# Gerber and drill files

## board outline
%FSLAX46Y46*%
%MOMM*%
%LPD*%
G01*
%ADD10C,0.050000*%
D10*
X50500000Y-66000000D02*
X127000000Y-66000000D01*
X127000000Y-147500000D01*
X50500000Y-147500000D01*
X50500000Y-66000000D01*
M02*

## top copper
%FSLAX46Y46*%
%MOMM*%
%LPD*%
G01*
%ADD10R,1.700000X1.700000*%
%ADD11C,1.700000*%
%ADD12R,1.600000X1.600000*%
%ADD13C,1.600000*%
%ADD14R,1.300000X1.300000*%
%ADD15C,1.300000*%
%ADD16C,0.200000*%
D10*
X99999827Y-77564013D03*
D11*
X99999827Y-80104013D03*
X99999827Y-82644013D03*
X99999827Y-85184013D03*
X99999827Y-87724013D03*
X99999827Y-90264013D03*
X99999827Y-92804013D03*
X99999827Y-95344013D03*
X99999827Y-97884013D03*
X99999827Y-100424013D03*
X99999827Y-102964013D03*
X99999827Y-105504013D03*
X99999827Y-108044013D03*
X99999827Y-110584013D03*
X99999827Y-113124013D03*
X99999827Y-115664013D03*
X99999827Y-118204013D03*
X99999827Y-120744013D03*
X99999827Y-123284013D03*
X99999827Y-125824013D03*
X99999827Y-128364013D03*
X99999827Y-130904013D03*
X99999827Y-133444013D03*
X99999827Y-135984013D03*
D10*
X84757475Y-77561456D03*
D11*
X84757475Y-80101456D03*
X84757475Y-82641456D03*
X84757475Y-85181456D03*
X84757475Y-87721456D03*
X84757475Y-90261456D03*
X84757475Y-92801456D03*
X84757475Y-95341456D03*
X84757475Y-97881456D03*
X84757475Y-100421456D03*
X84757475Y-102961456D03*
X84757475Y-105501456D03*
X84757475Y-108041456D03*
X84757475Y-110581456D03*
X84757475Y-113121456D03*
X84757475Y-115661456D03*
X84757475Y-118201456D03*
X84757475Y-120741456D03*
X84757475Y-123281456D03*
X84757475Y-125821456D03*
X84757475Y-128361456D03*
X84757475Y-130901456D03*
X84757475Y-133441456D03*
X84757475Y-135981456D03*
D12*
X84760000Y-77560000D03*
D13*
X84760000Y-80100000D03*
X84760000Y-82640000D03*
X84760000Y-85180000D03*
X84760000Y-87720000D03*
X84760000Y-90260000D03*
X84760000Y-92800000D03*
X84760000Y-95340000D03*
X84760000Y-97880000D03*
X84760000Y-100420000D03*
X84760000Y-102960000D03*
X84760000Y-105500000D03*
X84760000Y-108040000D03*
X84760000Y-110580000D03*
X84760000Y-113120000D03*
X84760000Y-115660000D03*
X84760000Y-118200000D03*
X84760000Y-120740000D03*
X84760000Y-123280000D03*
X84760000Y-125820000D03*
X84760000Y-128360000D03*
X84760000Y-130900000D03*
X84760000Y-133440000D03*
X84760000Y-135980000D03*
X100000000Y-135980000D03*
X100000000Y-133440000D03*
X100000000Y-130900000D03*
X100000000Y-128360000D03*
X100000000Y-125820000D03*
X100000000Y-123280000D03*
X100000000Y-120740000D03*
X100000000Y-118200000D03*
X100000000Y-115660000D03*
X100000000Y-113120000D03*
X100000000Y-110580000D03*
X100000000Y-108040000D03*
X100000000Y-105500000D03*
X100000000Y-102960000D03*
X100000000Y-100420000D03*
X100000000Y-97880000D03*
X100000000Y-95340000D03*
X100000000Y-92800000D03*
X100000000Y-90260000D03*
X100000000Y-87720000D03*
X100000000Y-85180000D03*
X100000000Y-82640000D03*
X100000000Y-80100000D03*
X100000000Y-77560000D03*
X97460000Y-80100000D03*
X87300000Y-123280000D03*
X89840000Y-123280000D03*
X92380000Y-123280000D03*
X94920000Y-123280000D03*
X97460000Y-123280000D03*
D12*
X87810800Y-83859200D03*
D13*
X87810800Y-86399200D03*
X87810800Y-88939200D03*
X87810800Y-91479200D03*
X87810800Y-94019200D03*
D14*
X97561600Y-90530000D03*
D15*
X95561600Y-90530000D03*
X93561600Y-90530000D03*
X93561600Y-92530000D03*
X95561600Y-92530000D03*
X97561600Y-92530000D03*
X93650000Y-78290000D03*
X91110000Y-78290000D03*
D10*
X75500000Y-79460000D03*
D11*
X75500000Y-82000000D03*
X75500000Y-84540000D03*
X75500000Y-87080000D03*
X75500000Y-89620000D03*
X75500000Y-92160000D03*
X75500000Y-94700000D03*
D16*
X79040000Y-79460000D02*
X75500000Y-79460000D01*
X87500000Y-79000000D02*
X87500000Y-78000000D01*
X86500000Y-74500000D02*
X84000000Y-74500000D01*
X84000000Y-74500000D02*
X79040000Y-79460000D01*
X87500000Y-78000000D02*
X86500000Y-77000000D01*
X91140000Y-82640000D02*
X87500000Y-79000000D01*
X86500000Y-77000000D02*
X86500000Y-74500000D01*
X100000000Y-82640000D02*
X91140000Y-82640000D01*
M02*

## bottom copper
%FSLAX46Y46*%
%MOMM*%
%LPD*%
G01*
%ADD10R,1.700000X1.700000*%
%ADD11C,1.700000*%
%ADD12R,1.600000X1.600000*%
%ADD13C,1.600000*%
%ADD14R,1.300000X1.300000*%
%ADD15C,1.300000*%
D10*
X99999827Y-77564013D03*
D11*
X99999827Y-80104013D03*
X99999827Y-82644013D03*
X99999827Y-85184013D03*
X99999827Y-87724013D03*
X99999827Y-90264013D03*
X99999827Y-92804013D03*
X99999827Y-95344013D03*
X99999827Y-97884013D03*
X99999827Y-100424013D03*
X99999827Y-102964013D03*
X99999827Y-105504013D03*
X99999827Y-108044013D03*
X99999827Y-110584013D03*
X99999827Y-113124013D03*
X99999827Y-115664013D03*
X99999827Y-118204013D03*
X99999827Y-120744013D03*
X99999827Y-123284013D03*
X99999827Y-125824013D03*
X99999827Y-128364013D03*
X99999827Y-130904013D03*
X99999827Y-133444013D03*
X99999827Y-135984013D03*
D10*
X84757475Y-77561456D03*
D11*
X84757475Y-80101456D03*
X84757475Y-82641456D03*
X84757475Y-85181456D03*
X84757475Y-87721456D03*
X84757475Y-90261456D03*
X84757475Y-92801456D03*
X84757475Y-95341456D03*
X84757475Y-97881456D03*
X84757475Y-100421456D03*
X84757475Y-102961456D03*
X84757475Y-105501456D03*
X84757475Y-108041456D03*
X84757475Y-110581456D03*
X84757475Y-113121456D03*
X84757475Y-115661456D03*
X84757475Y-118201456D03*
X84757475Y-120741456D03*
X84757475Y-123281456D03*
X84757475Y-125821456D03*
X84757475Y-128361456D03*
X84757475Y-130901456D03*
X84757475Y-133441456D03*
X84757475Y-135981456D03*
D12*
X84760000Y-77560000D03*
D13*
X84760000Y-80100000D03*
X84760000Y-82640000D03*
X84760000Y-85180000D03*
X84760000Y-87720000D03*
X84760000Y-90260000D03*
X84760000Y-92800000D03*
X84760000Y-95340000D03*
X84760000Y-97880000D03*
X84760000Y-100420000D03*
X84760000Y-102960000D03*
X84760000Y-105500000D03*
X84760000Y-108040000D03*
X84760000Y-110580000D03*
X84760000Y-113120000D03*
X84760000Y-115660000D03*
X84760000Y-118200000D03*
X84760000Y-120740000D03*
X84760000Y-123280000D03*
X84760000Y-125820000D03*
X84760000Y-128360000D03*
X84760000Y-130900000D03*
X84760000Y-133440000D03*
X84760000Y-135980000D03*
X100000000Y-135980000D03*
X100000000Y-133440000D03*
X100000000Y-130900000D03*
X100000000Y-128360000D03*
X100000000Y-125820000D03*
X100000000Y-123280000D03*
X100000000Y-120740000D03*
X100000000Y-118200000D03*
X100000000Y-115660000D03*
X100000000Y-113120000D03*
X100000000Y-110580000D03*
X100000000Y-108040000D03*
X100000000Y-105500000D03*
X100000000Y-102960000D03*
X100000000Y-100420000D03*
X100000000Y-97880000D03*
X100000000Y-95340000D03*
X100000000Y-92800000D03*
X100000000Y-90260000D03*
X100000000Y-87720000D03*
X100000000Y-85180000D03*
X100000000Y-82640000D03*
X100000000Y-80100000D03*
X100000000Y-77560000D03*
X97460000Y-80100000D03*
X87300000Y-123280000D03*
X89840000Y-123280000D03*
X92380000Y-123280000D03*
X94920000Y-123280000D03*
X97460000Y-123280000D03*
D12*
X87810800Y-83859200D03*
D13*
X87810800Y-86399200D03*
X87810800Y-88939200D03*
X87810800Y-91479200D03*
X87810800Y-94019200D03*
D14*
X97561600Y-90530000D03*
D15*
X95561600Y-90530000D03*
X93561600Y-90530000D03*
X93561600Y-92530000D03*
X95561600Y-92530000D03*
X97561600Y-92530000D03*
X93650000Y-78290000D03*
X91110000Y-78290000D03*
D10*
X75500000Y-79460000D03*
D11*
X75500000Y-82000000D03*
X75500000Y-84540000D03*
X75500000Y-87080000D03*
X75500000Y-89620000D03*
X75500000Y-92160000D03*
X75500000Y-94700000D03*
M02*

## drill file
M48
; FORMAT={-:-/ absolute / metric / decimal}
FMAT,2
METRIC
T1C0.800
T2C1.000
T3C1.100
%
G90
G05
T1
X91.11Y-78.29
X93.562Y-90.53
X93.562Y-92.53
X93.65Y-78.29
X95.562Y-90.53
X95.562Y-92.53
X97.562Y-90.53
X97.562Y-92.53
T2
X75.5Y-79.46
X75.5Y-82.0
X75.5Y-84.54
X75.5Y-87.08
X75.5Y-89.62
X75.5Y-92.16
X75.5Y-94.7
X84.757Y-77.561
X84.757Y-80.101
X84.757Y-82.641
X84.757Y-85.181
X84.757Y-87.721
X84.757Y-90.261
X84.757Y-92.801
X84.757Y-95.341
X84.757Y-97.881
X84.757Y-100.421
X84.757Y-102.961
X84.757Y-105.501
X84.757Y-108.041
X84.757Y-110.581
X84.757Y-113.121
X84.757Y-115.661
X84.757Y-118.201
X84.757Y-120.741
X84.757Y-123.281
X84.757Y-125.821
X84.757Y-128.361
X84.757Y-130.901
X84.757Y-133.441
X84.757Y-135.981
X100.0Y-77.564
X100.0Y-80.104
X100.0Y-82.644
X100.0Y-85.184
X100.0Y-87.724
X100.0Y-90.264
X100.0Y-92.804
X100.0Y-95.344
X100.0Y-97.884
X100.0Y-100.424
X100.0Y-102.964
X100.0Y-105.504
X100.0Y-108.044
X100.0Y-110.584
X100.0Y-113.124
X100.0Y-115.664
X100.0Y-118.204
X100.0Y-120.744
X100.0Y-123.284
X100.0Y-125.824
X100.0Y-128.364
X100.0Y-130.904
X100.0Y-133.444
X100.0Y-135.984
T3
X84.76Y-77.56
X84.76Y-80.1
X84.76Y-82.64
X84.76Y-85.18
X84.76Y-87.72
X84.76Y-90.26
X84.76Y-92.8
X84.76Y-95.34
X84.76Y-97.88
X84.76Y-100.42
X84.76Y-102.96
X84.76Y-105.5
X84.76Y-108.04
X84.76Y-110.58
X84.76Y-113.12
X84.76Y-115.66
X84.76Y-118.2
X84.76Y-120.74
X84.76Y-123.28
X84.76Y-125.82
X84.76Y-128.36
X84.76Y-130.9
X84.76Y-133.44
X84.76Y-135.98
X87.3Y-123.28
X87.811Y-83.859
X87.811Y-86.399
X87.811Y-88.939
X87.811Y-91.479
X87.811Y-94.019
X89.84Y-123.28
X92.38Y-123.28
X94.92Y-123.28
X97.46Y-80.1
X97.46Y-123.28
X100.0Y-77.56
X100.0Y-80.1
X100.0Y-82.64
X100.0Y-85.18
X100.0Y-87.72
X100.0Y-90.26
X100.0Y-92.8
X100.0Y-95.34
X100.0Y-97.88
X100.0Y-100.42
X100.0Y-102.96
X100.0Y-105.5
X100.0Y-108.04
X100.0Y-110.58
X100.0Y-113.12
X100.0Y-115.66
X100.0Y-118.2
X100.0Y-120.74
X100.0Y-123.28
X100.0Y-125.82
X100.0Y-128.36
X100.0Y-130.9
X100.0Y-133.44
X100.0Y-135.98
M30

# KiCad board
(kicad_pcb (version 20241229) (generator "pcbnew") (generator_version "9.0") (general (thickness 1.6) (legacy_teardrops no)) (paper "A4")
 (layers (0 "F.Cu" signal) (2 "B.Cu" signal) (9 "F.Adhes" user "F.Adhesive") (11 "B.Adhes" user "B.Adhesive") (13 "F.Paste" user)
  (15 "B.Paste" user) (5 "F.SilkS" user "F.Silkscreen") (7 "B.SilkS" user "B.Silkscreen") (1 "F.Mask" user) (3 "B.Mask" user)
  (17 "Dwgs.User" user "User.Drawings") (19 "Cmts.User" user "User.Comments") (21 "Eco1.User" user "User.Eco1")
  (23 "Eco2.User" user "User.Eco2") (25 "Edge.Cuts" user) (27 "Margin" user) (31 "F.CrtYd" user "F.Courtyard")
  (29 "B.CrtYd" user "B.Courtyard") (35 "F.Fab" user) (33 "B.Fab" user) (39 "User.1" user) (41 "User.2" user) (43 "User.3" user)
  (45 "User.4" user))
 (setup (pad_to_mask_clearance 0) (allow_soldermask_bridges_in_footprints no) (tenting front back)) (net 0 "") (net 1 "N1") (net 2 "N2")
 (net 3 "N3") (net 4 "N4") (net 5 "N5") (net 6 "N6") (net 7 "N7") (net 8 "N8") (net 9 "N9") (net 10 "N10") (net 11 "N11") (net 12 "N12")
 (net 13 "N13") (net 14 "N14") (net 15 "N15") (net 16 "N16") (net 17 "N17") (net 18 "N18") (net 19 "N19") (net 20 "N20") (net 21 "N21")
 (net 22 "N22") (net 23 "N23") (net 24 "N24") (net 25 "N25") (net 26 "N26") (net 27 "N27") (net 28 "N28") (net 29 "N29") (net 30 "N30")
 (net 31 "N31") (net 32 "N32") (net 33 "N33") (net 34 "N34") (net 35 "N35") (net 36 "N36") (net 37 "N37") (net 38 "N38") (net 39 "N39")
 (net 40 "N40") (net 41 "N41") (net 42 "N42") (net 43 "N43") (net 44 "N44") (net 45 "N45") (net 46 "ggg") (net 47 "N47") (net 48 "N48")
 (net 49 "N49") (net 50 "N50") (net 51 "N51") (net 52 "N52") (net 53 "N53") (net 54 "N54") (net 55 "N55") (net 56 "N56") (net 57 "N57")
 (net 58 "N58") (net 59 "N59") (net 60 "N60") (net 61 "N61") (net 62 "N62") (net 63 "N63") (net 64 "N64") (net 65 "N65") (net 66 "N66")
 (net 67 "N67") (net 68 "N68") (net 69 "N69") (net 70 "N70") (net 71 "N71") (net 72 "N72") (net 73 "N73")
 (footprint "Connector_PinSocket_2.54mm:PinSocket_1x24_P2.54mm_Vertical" (layer "F.Cu") (at 99.999827 77.564013)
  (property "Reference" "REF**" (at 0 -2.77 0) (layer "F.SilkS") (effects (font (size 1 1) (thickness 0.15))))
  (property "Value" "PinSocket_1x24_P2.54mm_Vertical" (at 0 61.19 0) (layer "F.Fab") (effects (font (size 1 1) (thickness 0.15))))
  (pad "1" thru_hole rect (at 0 0) (size 1.7 1.7) (drill 1) (layers "*.Cu" "*.Mask") (remove_unused_layers no))
  (pad "2" thru_hole circle (at 0 2.54) (size 1.7 1.7) (drill 1) (layers "*.Cu" "*.Mask") (remove_unused_layers no))
  (pad "3" thru_hole circle (at 0 5.08) (size 1.7 1.7) (drill 1) (layers "*.Cu" "*.Mask") (remove_unused_layers no))
  (pad "4" thru_hole circle (at 0 7.62) (size 1.7 1.7) (drill 1) (layers "*.Cu" "*.Mask") (remove_unused_layers no))
  (pad "5" thru_hole circle (at 0 10.16) (size 1.7 1.7) (drill 1) (layers "*.Cu" "*.Mask") (remove_unused_layers no))
  (pad "6" thru_hole circle (at 0 12.7) (size 1.7 1.7) (drill 1) (layers "*.Cu" "*.Mask") (remove_unused_layers no))
  (pad "7" thru_hole circle (at 0 15.24) (size 1.7 1.7) (drill 1) (layers "*.Cu" "*.Mask") (remove_unused_layers no))
  (pad "8" thru_hole circle (at 0 17.78) (size 1.7 1.7) (drill 1) (layers "*.Cu" "*.Mask") (remove_unused_layers no))
  (pad "9" thru_hole circle (at 0 20.32) (size 1.7 1.7) (drill 1) (layers "*.Cu" "*.Mask") (remove_unused_layers no))
  (pad "10" thru_hole circle (at 0 22.86) (size 1.7 1.7) (drill 1) (layers "*.Cu" "*.Mask") (remove_unused_layers no))
  (pad "11" thru_hole circle (at 0 25.4) (size 1.7 1.7) (drill 1) (layers "*.Cu" "*.Mask") (remove_unused_layers no))
  (pad "12" thru_hole circle (at 0 27.94) (size 1.7 1.7) (drill 1) (layers "*.Cu" "*.Mask") (remove_unused_layers no))
  (pad "13" thru_hole circle (at 0 30.48) (size 1.7 1.7) (drill 1) (layers "*.Cu" "*.Mask") (remove_unused_layers no))
  (pad "14" thru_hole circle (at 0 33.02) (size 1.7 1.7) (drill 1) (layers "*.Cu" "*.Mask") (remove_unused_layers no))
  (pad "15" thru_hole circle (at 0 35.56) (size 1.7 1.7) (drill 1) (layers "*.Cu" "*.Mask") (remove_unused_layers no))
  (pad "16" thru_hole circle (at 0 38.1) (size 1.7 1.7) (drill 1) (layers "*.Cu" "*.Mask") (remove_unused_layers no))
  (pad "17" thru_hole circle (at 0 40.64) (size 1.7 1.7) (drill 1) (layers "*.Cu" "*.Mask") (remove_unused_layers no))
  (pad "18" thru_hole circle (at 0 43.18) (size 1.7 1.7) (drill 1) (layers "*.Cu" "*.Mask") (remove_unused_layers no))
  (pad "19" thru_hole circle (at 0 45.72) (size 1.7 1.7) (drill 1) (layers "*.Cu" "*.Mask") (remove_unused_layers no))
  (pad "20" thru_hole circle (at 0 48.26) (size 1.7 1.7) (drill 1) (layers "*.Cu" "*.Mask") (remove_unused_layers no))
  (pad "21" thru_hole circle (at 0 50.8) (size 1.7 1.7) (drill 1) (layers "*.Cu" "*.Mask") (remove_unused_layers no))
  (pad "22" thru_hole circle (at 0 53.34) (size 1.7 1.7) (drill 1) (layers "*.Cu" "*.Mask") (remove_unused_layers no))
  (pad "23" thru_hole circle (at 0 55.88) (size 1.7 1.7) (drill 1) (layers "*.Cu" "*.Mask") (remove_unused_layers no))
  (pad "24" thru_hole circle (at 0 58.42) (size 1.7 1.7) (drill 1) (layers "*.Cu" "*.Mask") (remove_unused_layers no)))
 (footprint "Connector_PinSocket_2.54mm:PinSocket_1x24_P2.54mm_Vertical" (layer "F.Cu") (at 84.757475 77.561456)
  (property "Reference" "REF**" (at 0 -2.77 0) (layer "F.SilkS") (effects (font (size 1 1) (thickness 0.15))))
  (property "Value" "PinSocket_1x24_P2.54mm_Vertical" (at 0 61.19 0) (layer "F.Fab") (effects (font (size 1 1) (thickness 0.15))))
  (pad "1" thru_hole rect (at 0 0) (size 1.7 1.7) (drill 1) (layers "*.Cu" "*.Mask") (remove_unused_layers no))
  (pad "2" thru_hole circle (at 0 2.54) (size 1.7 1.7) (drill 1) (layers "*.Cu" "*.Mask") (remove_unused_layers no))
  (pad "3" thru_hole circle (at 0 5.08) (size 1.7 1.7) (drill 1) (layers "*.Cu" "*.Mask") (remove_unused_layers no))
  (pad "4" thru_hole circle (at 0 7.62) (size 1.7 1.7) (drill 1) (layers "*.Cu" "*.Mask") (remove_unused_layers no))
  (pad "5" thru_hole circle (at 0 10.16) (size 1.7 1.7) (drill 1) (layers "*.Cu" "*.Mask") (remove_unused_layers no))
  (pad "6" thru_hole circle (at 0 12.7) (size 1.7 1.7) (drill 1) (layers "*.Cu" "*.Mask") (remove_unused_layers no))
  (pad "7" thru_hole circle (at 0 15.24) (size 1.7 1.7) (drill 1) (layers "*.Cu" "*.Mask") (remove_unused_layers no))
  (pad "8" thru_hole circle (at 0 17.78) (size 1.7 1.7) (drill 1) (layers "*.Cu" "*.Mask") (remove_unused_layers no))
  (pad "9" thru_hole circle (at 0 20.32) (size 1.7 1.7) (drill 1) (layers "*.Cu" "*.Mask") (remove_unused_layers no))
  (pad "10" thru_hole circle (at 0 22.86) (size 1.7 1.7) (drill 1) (layers "*.Cu" "*.Mask") (remove_unused_layers no))
  (pad "11" thru_hole circle (at 0 25.4) (size 1.7 1.7) (drill 1) (layers "*.Cu" "*.Mask") (remove_unused_layers no))
  (pad "12" thru_hole circle (at 0 27.94) (size 1.7 1.7) (drill 1) (layers "*.Cu" "*.Mask") (remove_unused_layers no))
  (pad "13" thru_hole circle (at 0 30.48) (size 1.7 1.7) (drill 1) (layers "*.Cu" "*.Mask") (remove_unused_layers no))
  (pad "14" thru_hole circle (at 0 33.02) (size 1.7 1.7) (drill 1) (layers "*.Cu" "*.Mask") (remove_unused_layers no))
  (pad "15" thru_hole circle (at 0 35.56) (size 1.7 1.7) (drill 1) (layers "*.Cu" "*.Mask") (remove_unused_layers no))
  (pad "16" thru_hole circle (at 0 38.1) (size 1.7 1.7) (drill 1) (layers "*.Cu" "*.Mask") (remove_unused_layers no))
  (pad "17" thru_hole circle (at 0 40.64) (size 1.7 1.7) (drill 1) (layers "*.Cu" "*.Mask") (remove_unused_layers no))
  (pad "18" thru_hole circle (at 0 43.18) (size 1.7 1.7) (drill 1) (layers "*.Cu" "*.Mask") (remove_unused_layers no))
  (pad "19" thru_hole circle (at 0 45.72) (size 1.7 1.7) (drill 1) (layers "*.Cu" "*.Mask") (remove_unused_layers no))
  (pad "20" thru_hole circle (at 0 48.26) (size 1.7 1.7) (drill 1) (layers "*.Cu" "*.Mask") (remove_unused_layers no))
  (pad "21" thru_hole circle (at 0 50.8) (size 1.7 1.7) (drill 1) (layers "*.Cu" "*.Mask") (remove_unused_layers no))
  (pad "22" thru_hole circle (at 0 53.34) (size 1.7 1.7) (drill 1) (layers "*.Cu" "*.Mask") (remove_unused_layers no))
  (pad "23" thru_hole circle (at 0 55.88) (size 1.7 1.7) (drill 1) (layers "*.Cu" "*.Mask") (remove_unused_layers no))
  (pad "24" thru_hole circle (at 0 58.42) (size 1.7 1.7) (drill 1) (layers "*.Cu" "*.Mask") (remove_unused_layers no)))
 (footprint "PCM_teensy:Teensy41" (layer "F.Cu") (at 92.38 106.77 -90)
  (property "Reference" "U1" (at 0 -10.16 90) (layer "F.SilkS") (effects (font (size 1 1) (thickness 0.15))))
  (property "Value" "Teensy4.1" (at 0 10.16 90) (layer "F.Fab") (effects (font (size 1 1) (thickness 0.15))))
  (pad "1" thru_hole rect (at -29.21 7.62 270) (size 1.6 1.6) (drill 1.1) (layers "*.Cu" "*.Mask") (remove_unused_layers no) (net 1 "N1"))
  (pad "2" thru_hole circle (at -26.67 7.62 270) (size 1.6 1.6) (drill 1.1) (layers "*.Cu" "*.Mask") (remove_unused_layers no) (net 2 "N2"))
  (pad "3" thru_hole circle (at -24.13 7.62 270) (size 1.6 1.6) (drill 1.1) (layers "*.Cu" "*.Mask") (remove_unused_layers no) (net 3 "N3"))
  (pad "4" thru_hole circle (at -21.59 7.62 270) (size 1.6 1.6) (drill 1.1) (layers "*.Cu" "*.Mask") (remove_unused_layers no) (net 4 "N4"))
  (pad "5" thru_hole circle (at -19.05 7.62 270) (size 1.6 1.6) (drill 1.1) (layers "*.Cu" "*.Mask") (remove_unused_layers no) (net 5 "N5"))
  (pad "6" thru_hole circle (at -16.51 7.62 270) (size 1.6 1.6) (drill 1.1) (layers "*.Cu" "*.Mask") (remove_unused_layers no) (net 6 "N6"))
  (pad "7" thru_hole circle (at -13.97 7.62 270) (size 1.6 1.6) (drill 1.1) (layers "*.Cu" "*.Mask") (remove_unused_layers no) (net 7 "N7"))
  (pad "8" thru_hole circle (at -11.43 7.62 270) (size 1.6 1.6) (drill 1.1) (layers "*.Cu" "*.Mask") (remove_unused_layers no) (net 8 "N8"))
  (pad "9" thru_hole circle (at -8.89 7.62 270) (size 1.6 1.6) (drill 1.1) (layers "*.Cu" "*.Mask") (remove_unused_layers no) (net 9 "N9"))
  (pad "10" thru_hole circle (at -6.35 7.62 270) (size 1.6 1.6) (drill 1.1) (layers "*.Cu" "*.Mask") (remove_unused_layers no)
   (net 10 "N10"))
  (pad "11" thru_hole circle (at -3.81 7.62 270) (size 1.6 1.6) (drill 1.1) (layers "*.Cu" "*.Mask") (remove_unused_layers no)
   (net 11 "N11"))
  (pad "12" thru_hole circle (at -1.27 7.62 270) (size 1.6 1.6) (drill 1.1) (layers "*.Cu" "*.Mask") (remove_unused_layers no)
   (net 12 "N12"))
  (pad "13" thru_hole circle (at 1.27 7.62 270) (size 1.6 1.6) (drill 1.1) (layers "*.Cu" "*.Mask") (remove_unused_layers no) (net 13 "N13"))
  (pad "14" thru_hole circle (at 3.81 7.62 270) (size 1.6 1.6) (drill 1.1) (layers "*.Cu" "*.Mask") (remove_unused_layers no) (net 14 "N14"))
  (pad "15" thru_hole circle (at 6.35 7.62 270) (size 1.6 1.6) (drill 1.1) (layers "*.Cu" "*.Mask") (remove_unused_layers no) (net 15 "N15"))
  (pad "16" thru_hole circle (at 8.89 7.62 270) (size 1.6 1.6) (drill 1.1) (layers "*.Cu" "*.Mask") (remove_unused_layers no) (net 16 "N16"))
  (pad "17" thru_hole circle (at 11.43 7.62 270) (size 1.6 1.6) (drill 1.1) (layers "*.Cu" "*.Mask") (remove_unused_layers no)
   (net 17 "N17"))
  (pad "18" thru_hole circle (at 13.97 7.62 270) (size 1.6 1.6) (drill 1.1) (layers "*.Cu" "*.Mask") (remove_unused_layers no)
   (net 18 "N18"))
  (pad "19" thru_hole circle (at 16.51 7.62 270) (size 1.6 1.6) (drill 1.1) (layers "*.Cu" "*.Mask") (remove_unused_layers no)
   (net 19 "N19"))
  (pad "20" thru_hole circle (at 19.05 7.62 270) (size 1.6 1.6) (drill 1.1) (layers "*.Cu" "*.Mask") (remove_unused_layers no)
   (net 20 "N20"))
  (pad "21" thru_hole circle (at 21.59 7.62 270) (size 1.6 1.6) (drill 1.1) (layers "*.Cu" "*.Mask") (remove_unused_layers no)
   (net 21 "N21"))
  (pad "22" thru_hole circle (at 24.13 7.62 270) (size 1.6 1.6) (drill 1.1) (layers "*.Cu" "*.Mask") (remove_unused_layers no)
   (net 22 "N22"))
  (pad "23" thru_hole circle (at 26.67 7.62 270) (size 1.6 1.6) (drill 1.1) (layers "*.Cu" "*.Mask") (remove_unused_layers no)
   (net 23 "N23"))
  (pad "24" thru_hole circle (at 29.21 7.62 270) (size 1.6 1.6) (drill 1.1) (layers "*.Cu" "*.Mask") (remove_unused_layers no)
   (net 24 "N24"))
  (pad "25" thru_hole circle (at 29.21 -7.62 270) (size 1.6 1.6) (drill 1.1) (layers "*.Cu" "*.Mask") (remove_unused_layers no)
   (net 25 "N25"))
  (pad "26" thru_hole circle (at 26.67 -7.62 270) (size 1.6 1.6) (drill 1.1) (layers "*.Cu" "*.Mask") (remove_unused_layers no)
   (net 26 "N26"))
  (pad "27" thru_hole circle (at 24.13 -7.62 270) (size 1.6 1.6) (drill 1.1) (layers "*.Cu" "*.Mask") (remove_unused_layers no)
   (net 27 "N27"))
  (pad "28" thru_hole circle (at 21.59 -7.62 270) (size 1.6 1.6) (drill 1.1) (layers "*.Cu" "*.Mask") (remove_unused_layers no)
   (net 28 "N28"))
  (pad "29" thru_hole circle (at 19.05 -7.62 270) (size 1.6 1.6) (drill 1.1) (layers "*.Cu" "*.Mask") (remove_unused_layers no)
   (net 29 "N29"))
  (pad "30" thru_hole circle (at 16.51 -7.62 270) (size 1.6 1.6) (drill 1.1) (layers "*.Cu" "*.Mask") (remove_unused_layers no)
   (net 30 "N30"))
  (pad "31" thru_hole circle (at 13.97 -7.62 270) (size 1.6 1.6) (drill 1.1) (layers "*.Cu" "*.Mask") (remove_unused_layers no)
   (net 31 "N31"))
  (pad "32" thru_hole circle (at 11.43 -7.62 270) (size 1.6 1.6) (drill 1.1) (layers "*.Cu" "*.Mask") (remove_unused_layers no)
   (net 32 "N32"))
  (pad "33" thru_hole circle (at 8.89 -7.62 270) (size 1.6 1.6) (drill 1.1) (layers "*.Cu" "*.Mask") (remove_unused_layers no)
   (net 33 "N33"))
  (pad "34" thru_hole circle (at 6.35 -7.62 270) (size 1.6 1.6) (drill 1.1) (layers "*.Cu" "*.Mask") (remove_unused_layers no)
   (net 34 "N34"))
  (pad "35" thru_hole circle (at 3.81 -7.62 270) (size 1.6 1.6) (drill 1.1) (layers "*.Cu" "*.Mask") (remove_unused_layers no)
   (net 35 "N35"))
  (pad "36" thru_hole circle (at 1.27 -7.62 270) (size 1.6 1.6) (drill 1.1) (layers "*.Cu" "*.Mask") (remove_unused_layers no)
   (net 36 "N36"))
  (pad "37" thru_hole circle (at -1.27 -7.62 270) (size 1.6 1.6) (drill 1.1) (layers "*.Cu" "*.Mask") (remove_unused_layers no)
   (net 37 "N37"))
  (pad "38" thru_hole circle (at -3.81 -7.62 270) (size 1.6 1.6) (drill 1.1) (layers "*.Cu" "*.Mask") (remove_unused_layers no)
   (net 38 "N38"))
  (pad "39" thru_hole circle (at -6.35 -7.62 270) (size 1.6 1.6) (drill 1.1) (layers "*.Cu" "*.Mask") (remove_unused_layers no)
   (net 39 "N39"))
  (pad "40" thru_hole circle (at -8.89 -7.62 270) (size 1.6 1.6) (drill 1.1) (layers "*.Cu" "*.Mask") (remove_unused_layers no)
   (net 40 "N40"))
  (pad "41" thru_hole circle (at -11.43 -7.62 270) (size 1.6 1.6) (drill 1.1) (layers "*.Cu" "*.Mask") (remove_unused_layers no)
   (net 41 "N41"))
  (pad "42" thru_hole circle (at -13.97 -7.62 270) (size 1.6 1.6) (drill 1.1) (layers "*.Cu" "*.Mask") (remove_unused_layers no)
   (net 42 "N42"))
  (pad "43" thru_hole circle (at -16.51 -7.62 270) (size 1.6 1.6) (drill 1.1) (layers "*.Cu" "*.Mask") (remove_unused_layers no)
   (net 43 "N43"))
  (pad "44" thru_hole circle (at -19.05 -7.62 270) (size 1.6 1.6) (drill 1.1) (layers "*.Cu" "*.Mask") (remove_unused_layers no)
   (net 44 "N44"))
  (pad "45" thru_hole circle (at -21.59 -7.62 270) (size 1.6 1.6) (drill 1.1) (layers "*.Cu" "*.Mask") (remove_unused_layers no)
   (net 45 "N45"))
  (pad "46" thru_hole circle (at -24.13 -7.62 270) (size 1.6 1.6) (drill 1.1) (layers "*.Cu" "*.Mask") (remove_unused_layers no)
   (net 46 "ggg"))
  (pad "47" thru_hole circle (at -26.67 -7.62 270) (size 1.6 1.6) (drill 1.1) (layers "*.Cu" "*.Mask") (remove_unused_layers no)
   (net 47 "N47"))
  (pad "48" thru_hole circle (at -29.21 -7.62 270) (size 1.6 1.6) (drill 1.1) (layers "*.Cu" "*.Mask") (remove_unused_layers no)
   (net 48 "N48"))
  (pad "49" thru_hole circle (at -26.67 -5.08 270) (size 1.6 1.6) (drill 1.1) (layers "*.Cu" "*.Mask") (remove_unused_layers no)
   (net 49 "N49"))
  (pad "50" thru_hole circle (at 16.51 5.08 270) (size 1.6 1.6) (drill 1.1) (layers "*.Cu" "*.Mask") (remove_unused_layers no)
   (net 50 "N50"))
  (pad "51" thru_hole circle (at 16.51 2.54 270) (size 1.6 1.6) (drill 1.1) (layers "*.Cu" "*.Mask") (remove_unused_layers no)
   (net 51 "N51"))
  (pad "52" thru_hole circle (at 16.51 0 270) (size 1.6 1.6) (drill 1.1) (layers "*.Cu" "*.Mask") (remove_unused_layers no) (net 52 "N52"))
  (pad "53" thru_hole circle (at 16.51 -2.54 270) (size 1.6 1.6) (drill 1.1) (layers "*.Cu" "*.Mask") (remove_unused_layers no)
   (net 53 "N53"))
  (pad "54" thru_hole circle (at 16.51 -5.08 270) (size 1.6 1.6) (drill 1.1) (layers "*.Cu" "*.Mask") (remove_unused_layers no)
   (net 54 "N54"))
  (pad "55" thru_hole rect (at -22.9108 4.5692 270) (size 1.6 1.6) (drill 1.1) (layers "*.Cu" "*.Mask") (remove_unused_layers no)
   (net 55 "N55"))
  (pad "56" thru_hole circle (at -20.3708 4.5692 270) (size 1.6 1.6) (drill 1.1) (layers "*.Cu" "*.Mask") (remove_unused_layers no)
   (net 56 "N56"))
  (pad "57" thru_hole circle (at -17.8308 4.5692 270) (size 1.6 1.6) (drill 1.1) (layers "*.Cu" "*.Mask") (remove_unused_layers no)
   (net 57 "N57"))
  (pad "58" thru_hole circle (at -15.2908 4.5692 270) (size 1.6 1.6) (drill 1.1) (layers "*.Cu" "*.Mask") (remove_unused_layers no)
   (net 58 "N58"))
  (pad "59" thru_hole circle (at -12.7508 4.5692 270) (size 1.6 1.6) (drill 1.1) (layers "*.Cu" "*.Mask") (remove_unused_layers no)
   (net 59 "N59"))
  (pad "60" thru_hole rect (at -16.24 -5.1816 270) (size 1.3 1.3) (drill 0.8) (layers "*.Cu" "*.Mask") (remove_unused_layers no)
   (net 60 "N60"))
  (pad "61" thru_hole circle (at -16.24 -3.1816 270) (size 1.3 1.3) (drill 0.8) (layers "*.Cu" "*.Mask") (remove_unused_layers no)
   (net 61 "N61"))
  (pad "62" thru_hole circle (at -16.24 -1.1816 270) (size 1.3 1.3) (drill 0.8) (layers "*.Cu" "*.Mask") (remove_unused_layers no)
   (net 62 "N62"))
  (pad "63" thru_hole circle (at -14.24 -1.1816 270) (size 1.3 1.3) (drill 0.8) (layers "*.Cu" "*.Mask") (remove_unused_layers no)
   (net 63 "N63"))
  (pad "64" thru_hole circle (at -14.24 -3.1816 270) (size 1.3 1.3) (drill 0.8) (layers "*.Cu" "*.Mask") (remove_unused_layers no)
   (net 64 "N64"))
  (pad "65" thru_hole circle (at -14.24 -5.1816 270) (size 1.3 1.3) (drill 0.8) (layers "*.Cu" "*.Mask") (remove_unused_layers no)
   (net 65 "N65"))
  (pad "66" thru_hole circle (at -28.48 -1.27 270) (size 1.3 1.3) (drill 0.8) (layers "*.Cu" "*.Mask") (remove_unused_layers no)
   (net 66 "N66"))
  (pad "67" thru_hole circle (at -28.48 1.27 270) (size 1.3 1.3) (drill 0.8) (layers "*.Cu" "*.Mask") (remove_unused_layers no)
   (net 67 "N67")))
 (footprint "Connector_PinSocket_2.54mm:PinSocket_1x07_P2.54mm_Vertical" (layer "F.Cu") (at 75.5 79.46)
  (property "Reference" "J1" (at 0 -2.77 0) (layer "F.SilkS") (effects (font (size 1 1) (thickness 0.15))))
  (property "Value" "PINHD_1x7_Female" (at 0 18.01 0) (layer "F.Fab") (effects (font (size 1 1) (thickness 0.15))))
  (pad "1" thru_hole rect (at 0 0) (size 1.7 1.7) (drill 1) (layers "*.Cu" "*.Mask") (remove_unused_layers no) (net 46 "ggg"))
  (pad "2" thru_hole circle (at 0 2.54) (size 1.7 1.7) (drill 1) (layers "*.Cu" "*.Mask") (remove_unused_layers no) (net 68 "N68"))
  (pad "3" thru_hole circle (at 0 5.08) (size 1.7 1.7) (drill 1) (layers "*.Cu" "*.Mask") (remove_unused_layers no) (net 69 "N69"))
  (pad "4" thru_hole circle (at 0 7.62) (size 1.7 1.7) (drill 1) (layers "*.Cu" "*.Mask") (remove_unused_layers no) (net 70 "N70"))
  (pad "5" thru_hole circle (at 0 10.16) (size 1.7 1.7) (drill 1) (layers "*.Cu" "*.Mask") (remove_unused_layers no) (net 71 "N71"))
  (pad "6" thru_hole circle (at 0 12.7) (size 1.7 1.7) (drill 1) (layers "*.Cu" "*.Mask") (remove_unused_layers no) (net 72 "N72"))
  (pad "7" thru_hole circle (at 0 15.24) (size 1.7 1.7) (drill 1) (layers "*.Cu" "*.Mask") (remove_unused_layers no) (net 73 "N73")))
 (gr_rect (start 50.5 66) (end 127 147.5) (stroke (width 0.05) (type default)) (fill no) (layer "Edge.Cuts"))
 (segment (start 79.04 79.46) (end 75.5 79.46) (width 0.2) (layer "F.Cu") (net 46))
 (segment (start 87.5 79) (end 87.5 78) (width 0.2) (layer "F.Cu") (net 46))
 (segment (start 86.5 74.5) (end 84 74.5) (width 0.2) (layer "F.Cu") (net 46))
 (segment (start 84 74.5) (end 79.04 79.46) (width 0.2) (layer "F.Cu") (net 46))
 (segment (start 87.5 78) (end 86.5 77) (width 0.2) (layer "F.Cu") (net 46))
 (segment (start 91.14 82.64) (end 87.5 79) (width 0.2) (layer "F.Cu") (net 46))
 (segment (start 86.5 77) (end 86.5 74.5) (width 0.2) (layer "F.Cu") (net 46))
 (segment (start 100 82.64) (end 91.14 82.64) (width 0.2) (layer "F.Cu") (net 46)))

